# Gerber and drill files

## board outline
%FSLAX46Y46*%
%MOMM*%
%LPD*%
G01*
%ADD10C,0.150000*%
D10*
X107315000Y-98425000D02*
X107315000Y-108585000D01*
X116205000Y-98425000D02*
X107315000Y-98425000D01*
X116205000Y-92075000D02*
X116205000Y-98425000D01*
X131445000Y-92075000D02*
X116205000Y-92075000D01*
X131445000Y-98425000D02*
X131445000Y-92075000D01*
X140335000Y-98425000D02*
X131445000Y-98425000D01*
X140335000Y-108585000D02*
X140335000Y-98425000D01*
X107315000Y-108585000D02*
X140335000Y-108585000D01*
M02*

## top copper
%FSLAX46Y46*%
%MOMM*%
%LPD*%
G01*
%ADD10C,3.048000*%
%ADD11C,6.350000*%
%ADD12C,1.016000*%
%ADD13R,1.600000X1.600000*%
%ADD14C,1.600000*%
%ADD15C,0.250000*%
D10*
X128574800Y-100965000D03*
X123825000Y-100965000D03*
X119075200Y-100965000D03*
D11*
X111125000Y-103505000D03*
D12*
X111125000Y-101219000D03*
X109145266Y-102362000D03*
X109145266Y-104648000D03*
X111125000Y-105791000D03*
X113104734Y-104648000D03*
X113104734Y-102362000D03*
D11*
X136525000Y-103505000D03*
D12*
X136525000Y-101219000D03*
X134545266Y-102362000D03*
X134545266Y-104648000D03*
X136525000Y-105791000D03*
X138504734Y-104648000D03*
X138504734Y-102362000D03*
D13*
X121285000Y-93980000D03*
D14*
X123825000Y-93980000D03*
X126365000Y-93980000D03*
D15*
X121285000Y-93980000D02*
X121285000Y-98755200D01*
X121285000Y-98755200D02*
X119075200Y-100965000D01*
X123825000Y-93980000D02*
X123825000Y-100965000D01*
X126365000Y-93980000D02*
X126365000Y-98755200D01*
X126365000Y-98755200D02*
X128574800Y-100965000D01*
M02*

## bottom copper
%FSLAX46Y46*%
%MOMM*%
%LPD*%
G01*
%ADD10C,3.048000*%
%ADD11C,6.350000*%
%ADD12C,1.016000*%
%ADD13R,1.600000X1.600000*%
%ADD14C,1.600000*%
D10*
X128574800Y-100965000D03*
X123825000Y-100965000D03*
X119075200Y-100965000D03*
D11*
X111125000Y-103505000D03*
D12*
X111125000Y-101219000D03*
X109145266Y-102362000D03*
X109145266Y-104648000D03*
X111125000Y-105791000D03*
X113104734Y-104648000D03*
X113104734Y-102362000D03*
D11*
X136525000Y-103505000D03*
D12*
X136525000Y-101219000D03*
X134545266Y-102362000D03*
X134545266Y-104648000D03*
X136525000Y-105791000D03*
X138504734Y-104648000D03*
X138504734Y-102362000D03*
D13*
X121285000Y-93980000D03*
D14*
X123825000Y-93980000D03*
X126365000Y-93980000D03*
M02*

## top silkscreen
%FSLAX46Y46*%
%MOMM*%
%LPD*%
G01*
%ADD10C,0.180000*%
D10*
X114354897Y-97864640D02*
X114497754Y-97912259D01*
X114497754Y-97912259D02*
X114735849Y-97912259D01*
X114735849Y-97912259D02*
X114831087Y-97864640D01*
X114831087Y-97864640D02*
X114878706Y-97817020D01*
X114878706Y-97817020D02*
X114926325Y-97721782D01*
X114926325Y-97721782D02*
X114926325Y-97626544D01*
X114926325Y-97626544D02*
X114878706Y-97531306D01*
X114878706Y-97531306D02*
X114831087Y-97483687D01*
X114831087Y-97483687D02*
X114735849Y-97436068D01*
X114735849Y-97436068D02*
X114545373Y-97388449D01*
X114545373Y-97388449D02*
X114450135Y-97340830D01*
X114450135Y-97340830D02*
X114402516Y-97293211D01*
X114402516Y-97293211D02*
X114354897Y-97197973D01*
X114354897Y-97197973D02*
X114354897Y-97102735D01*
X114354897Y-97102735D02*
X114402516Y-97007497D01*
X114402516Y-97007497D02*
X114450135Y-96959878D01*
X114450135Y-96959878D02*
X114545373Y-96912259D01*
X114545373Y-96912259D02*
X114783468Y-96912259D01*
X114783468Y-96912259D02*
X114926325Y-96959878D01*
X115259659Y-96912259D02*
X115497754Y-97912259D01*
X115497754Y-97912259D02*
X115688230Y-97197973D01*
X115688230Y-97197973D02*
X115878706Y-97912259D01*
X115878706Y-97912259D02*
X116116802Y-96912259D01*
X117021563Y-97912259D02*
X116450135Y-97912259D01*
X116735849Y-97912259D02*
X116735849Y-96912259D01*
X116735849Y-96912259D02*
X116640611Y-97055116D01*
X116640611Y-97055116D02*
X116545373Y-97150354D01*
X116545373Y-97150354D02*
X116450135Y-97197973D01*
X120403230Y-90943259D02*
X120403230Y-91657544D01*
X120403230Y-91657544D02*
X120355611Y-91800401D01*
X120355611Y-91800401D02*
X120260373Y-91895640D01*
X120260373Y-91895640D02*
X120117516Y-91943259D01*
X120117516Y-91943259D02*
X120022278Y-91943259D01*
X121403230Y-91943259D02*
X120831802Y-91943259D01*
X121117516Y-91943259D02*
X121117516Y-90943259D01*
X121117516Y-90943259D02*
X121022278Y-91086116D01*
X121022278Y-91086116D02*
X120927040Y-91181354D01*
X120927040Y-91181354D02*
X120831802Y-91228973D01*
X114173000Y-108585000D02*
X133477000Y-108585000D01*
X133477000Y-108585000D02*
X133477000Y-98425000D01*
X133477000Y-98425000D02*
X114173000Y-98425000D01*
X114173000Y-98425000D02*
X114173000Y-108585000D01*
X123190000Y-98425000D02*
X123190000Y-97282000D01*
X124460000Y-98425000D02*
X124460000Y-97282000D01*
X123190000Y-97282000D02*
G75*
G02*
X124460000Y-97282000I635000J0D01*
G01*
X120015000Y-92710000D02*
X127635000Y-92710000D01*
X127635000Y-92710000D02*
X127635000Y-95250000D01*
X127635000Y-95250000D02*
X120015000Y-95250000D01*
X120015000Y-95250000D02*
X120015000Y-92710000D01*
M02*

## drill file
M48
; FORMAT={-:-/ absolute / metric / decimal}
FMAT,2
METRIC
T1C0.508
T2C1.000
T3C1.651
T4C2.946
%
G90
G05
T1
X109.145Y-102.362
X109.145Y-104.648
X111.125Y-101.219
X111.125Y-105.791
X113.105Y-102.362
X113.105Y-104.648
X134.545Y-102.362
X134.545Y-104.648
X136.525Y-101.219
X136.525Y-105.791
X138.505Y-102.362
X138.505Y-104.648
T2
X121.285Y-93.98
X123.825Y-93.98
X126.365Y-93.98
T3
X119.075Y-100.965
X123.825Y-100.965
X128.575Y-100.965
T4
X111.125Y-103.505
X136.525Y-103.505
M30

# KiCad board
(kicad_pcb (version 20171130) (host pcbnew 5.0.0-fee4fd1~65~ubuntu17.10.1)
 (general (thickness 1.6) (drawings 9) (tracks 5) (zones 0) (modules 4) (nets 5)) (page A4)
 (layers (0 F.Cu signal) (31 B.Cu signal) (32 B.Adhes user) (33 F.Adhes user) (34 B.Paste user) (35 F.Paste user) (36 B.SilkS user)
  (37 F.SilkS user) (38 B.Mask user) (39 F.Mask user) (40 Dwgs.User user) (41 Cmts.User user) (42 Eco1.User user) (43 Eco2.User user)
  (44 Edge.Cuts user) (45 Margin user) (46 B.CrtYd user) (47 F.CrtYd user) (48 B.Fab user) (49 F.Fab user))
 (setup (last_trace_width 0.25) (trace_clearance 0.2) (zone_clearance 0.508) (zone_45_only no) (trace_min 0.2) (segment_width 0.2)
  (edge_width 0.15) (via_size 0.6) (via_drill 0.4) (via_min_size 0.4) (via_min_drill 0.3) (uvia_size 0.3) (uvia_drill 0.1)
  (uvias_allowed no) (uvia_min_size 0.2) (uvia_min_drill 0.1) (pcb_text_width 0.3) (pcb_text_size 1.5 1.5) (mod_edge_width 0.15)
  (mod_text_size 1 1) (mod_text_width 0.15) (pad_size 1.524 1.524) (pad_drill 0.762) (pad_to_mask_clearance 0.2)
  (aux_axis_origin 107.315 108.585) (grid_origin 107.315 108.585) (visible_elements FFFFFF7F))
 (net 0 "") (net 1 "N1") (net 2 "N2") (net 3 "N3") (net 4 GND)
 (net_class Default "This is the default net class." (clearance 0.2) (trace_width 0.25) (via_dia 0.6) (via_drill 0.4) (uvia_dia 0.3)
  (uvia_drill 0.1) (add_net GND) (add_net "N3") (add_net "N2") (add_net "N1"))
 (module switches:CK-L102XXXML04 (layer F.Cu) (at 123.825 108.585)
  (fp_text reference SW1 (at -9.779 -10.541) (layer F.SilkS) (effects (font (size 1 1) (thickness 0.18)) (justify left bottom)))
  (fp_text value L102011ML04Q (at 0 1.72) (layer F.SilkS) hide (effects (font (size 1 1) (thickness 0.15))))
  (fp_line (start -9.652 0) (end 9.652 0) (layer F.SilkS) (width 0.18))
  (fp_line (start 9.652 0) (end 9.652 -10.16) (layer F.SilkS) (width 0.18))
  (fp_line (start 9.652 -10.16) (end -9.652 -10.16) (layer F.SilkS) (width 0.18))
  (fp_line (start -9.652 -10.16) (end -9.652 0) (layer F.SilkS) (width 0.18))
  (fp_line (start -0.635 -10.16) (end -0.635 -11.303) (layer F.SilkS) (width 0.18))
  (fp_line (start 0.635 -10.16) (end 0.635 -11.303) (layer F.SilkS) (width 0.18))
  (fp_arc (start 0 -11.303) (end -0.635 -11.303) (angle 180) (layer F.SilkS) (width 0.18))
  (pad 3 thru_hole circle (at 4.7498 -7.62) (size 3.048 3.048) (drill 1.651) (layers *.Cu *.Mask) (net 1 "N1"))
  (pad 2 thru_hole circle (at 0 -7.62) (size 3.048 3.048) (drill 1.651) (layers *.Cu *.Mask) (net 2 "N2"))
  (pad 1 thru_hole circle (at -4.7498 -7.62) (size 3.048 3.048) (drill 1.651) (layers *.Cu *.Mask) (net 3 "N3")))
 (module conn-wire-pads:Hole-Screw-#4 (layer F.Cu) (at 111.125 103.505)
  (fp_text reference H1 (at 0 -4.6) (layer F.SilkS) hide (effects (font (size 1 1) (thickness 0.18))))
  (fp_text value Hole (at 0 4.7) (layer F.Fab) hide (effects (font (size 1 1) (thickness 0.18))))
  (pad P thru_hole circle (at 0 0) (size 6.35 6.35) (drill 2.9464) (layers *.Cu *.Mask) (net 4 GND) (clearance 1.016) (zone_connect 2))
  (pad P thru_hole circle (at 0 -2.286) (size 1.016 1.016) (drill 0.508) (layers *.Cu) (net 4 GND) (zone_connect 2))
  (pad P thru_hole circle (at -1.979734 -1.143 60) (size 1.016 1.016) (drill 0.508) (layers *.Cu) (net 4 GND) (zone_connect 2))
  (pad P thru_hole circle (at -1.979734 1.143 120) (size 1.016 1.016) (drill 0.508) (layers *.Cu) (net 4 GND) (zone_connect 2))
  (pad P thru_hole circle (at 0 2.286 180) (size 1.016 1.016) (drill 0.508) (layers *.Cu) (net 4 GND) (zone_connect 2))
  (pad P thru_hole circle (at 1.979734 1.143 240) (size 1.016 1.016) (drill 0.508) (layers *.Cu) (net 4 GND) (zone_connect 2))
  (pad P thru_hole circle (at 1.979734 -1.143 300) (size 1.016 1.016) (drill 0.508) (layers *.Cu) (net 4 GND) (zone_connect 2)))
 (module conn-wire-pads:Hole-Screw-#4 (layer F.Cu) (at 136.525 103.505)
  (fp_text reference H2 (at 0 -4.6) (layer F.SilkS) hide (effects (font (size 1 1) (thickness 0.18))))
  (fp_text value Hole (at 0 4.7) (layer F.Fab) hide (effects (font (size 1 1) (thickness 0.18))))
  (pad P thru_hole circle (at 0 0) (size 6.35 6.35) (drill 2.9464) (layers *.Cu *.Mask) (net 4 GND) (clearance 1.016) (zone_connect 2))
  (pad P thru_hole circle (at 0 -2.286) (size 1.016 1.016) (drill 0.508) (layers *.Cu) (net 4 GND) (zone_connect 2))
  (pad P thru_hole circle (at -1.979734 -1.143 60) (size 1.016 1.016) (drill 0.508) (layers *.Cu) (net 4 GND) (zone_connect 2))
  (pad P thru_hole circle (at -1.979734 1.143 120) (size 1.016 1.016) (drill 0.508) (layers *.Cu) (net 4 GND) (zone_connect 2))
  (pad P thru_hole circle (at 0 2.286 180) (size 1.016 1.016) (drill 0.508) (layers *.Cu) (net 4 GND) (zone_connect 2))
  (pad P thru_hole circle (at 1.979734 1.143 240) (size 1.016 1.016) (drill 0.508) (layers *.Cu) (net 4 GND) (zone_connect 2))
  (pad P thru_hole circle (at 1.979734 -1.143 300) (size 1.016 1.016) (drill 0.508) (layers *.Cu) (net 4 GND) (zone_connect 2)))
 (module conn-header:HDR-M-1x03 (layer F.Cu) (at 123.825 93.98)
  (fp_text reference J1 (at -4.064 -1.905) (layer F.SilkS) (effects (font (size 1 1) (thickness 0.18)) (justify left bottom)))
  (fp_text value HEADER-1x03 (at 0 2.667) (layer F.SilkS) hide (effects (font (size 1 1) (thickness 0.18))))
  (fp_line (start -3.81 -1.27) (end 3.81 -1.27) (layer F.SilkS) (width 0.18))
  (fp_line (start 3.81 -1.27) (end 3.81 1.27) (layer F.SilkS) (width 0.18))
  (fp_line (start 3.81 1.27) (end -3.81 1.27) (layer F.SilkS) (width 0.18))
  (fp_line (start -3.81 1.27) (end -3.81 -1.27) (layer F.SilkS) (width 0.18))
  (pad 1 thru_hole rect (at -2.54 0) (size 1.6 1.6) (drill 1) (layers *.Cu *.Mask) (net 3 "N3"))
  (pad 2 thru_hole circle (at 0 0) (size 1.6 1.6) (drill 1) (layers *.Cu *.Mask) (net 2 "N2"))
  (pad 3 thru_hole circle (at 2.54 0) (size 1.6 1.6) (drill 1) (layers *.Cu *.Mask) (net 1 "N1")))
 (gr_line (start 107.315 98.425) (end 107.315 108.585) (layer Edge.Cuts) (width 0.15))
 (gr_line (start 116.205 98.425) (end 107.315 98.425) (layer Edge.Cuts) (width 0.15))
 (gr_line (start 116.205 92.075) (end 116.205 98.425) (layer Edge.Cuts) (width 0.15))
 (gr_line (start 131.445 92.075) (end 116.205 92.075) (layer Edge.Cuts) (width 0.15))
 (gr_line (start 131.445 98.425) (end 131.445 92.075) (layer Edge.Cuts) (width 0.15))
 (gr_line (start 140.335 98.425) (end 131.445 98.425) (layer Edge.Cuts) (width 0.15))
 (gr_line (start 140.335 108.585) (end 140.335 98.425) (layer Edge.Cuts) (width 0.15))
 (gr_line (start 107.315 108.585) (end 140.335 108.585) (layer Edge.Cuts) (width 0.15))
 (segment (start 121.285 93.98) (end 121.285 98.7552) (width 0.25) (layer F.Cu) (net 3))
 (segment (start 121.285 98.7552) (end 119.0752 100.965) (width 0.25) (layer F.Cu) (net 3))
 (segment (start 123.825 93.98) (end 123.825 100.965) (width 0.25) (layer F.Cu) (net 2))
 (segment (start 126.365 93.98) (end 126.365 98.7552) (width 0.25) (layer F.Cu) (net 1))
 (segment (start 126.365 98.7552) (end 128.5748 100.965) (width 0.25) (layer F.Cu) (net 1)))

